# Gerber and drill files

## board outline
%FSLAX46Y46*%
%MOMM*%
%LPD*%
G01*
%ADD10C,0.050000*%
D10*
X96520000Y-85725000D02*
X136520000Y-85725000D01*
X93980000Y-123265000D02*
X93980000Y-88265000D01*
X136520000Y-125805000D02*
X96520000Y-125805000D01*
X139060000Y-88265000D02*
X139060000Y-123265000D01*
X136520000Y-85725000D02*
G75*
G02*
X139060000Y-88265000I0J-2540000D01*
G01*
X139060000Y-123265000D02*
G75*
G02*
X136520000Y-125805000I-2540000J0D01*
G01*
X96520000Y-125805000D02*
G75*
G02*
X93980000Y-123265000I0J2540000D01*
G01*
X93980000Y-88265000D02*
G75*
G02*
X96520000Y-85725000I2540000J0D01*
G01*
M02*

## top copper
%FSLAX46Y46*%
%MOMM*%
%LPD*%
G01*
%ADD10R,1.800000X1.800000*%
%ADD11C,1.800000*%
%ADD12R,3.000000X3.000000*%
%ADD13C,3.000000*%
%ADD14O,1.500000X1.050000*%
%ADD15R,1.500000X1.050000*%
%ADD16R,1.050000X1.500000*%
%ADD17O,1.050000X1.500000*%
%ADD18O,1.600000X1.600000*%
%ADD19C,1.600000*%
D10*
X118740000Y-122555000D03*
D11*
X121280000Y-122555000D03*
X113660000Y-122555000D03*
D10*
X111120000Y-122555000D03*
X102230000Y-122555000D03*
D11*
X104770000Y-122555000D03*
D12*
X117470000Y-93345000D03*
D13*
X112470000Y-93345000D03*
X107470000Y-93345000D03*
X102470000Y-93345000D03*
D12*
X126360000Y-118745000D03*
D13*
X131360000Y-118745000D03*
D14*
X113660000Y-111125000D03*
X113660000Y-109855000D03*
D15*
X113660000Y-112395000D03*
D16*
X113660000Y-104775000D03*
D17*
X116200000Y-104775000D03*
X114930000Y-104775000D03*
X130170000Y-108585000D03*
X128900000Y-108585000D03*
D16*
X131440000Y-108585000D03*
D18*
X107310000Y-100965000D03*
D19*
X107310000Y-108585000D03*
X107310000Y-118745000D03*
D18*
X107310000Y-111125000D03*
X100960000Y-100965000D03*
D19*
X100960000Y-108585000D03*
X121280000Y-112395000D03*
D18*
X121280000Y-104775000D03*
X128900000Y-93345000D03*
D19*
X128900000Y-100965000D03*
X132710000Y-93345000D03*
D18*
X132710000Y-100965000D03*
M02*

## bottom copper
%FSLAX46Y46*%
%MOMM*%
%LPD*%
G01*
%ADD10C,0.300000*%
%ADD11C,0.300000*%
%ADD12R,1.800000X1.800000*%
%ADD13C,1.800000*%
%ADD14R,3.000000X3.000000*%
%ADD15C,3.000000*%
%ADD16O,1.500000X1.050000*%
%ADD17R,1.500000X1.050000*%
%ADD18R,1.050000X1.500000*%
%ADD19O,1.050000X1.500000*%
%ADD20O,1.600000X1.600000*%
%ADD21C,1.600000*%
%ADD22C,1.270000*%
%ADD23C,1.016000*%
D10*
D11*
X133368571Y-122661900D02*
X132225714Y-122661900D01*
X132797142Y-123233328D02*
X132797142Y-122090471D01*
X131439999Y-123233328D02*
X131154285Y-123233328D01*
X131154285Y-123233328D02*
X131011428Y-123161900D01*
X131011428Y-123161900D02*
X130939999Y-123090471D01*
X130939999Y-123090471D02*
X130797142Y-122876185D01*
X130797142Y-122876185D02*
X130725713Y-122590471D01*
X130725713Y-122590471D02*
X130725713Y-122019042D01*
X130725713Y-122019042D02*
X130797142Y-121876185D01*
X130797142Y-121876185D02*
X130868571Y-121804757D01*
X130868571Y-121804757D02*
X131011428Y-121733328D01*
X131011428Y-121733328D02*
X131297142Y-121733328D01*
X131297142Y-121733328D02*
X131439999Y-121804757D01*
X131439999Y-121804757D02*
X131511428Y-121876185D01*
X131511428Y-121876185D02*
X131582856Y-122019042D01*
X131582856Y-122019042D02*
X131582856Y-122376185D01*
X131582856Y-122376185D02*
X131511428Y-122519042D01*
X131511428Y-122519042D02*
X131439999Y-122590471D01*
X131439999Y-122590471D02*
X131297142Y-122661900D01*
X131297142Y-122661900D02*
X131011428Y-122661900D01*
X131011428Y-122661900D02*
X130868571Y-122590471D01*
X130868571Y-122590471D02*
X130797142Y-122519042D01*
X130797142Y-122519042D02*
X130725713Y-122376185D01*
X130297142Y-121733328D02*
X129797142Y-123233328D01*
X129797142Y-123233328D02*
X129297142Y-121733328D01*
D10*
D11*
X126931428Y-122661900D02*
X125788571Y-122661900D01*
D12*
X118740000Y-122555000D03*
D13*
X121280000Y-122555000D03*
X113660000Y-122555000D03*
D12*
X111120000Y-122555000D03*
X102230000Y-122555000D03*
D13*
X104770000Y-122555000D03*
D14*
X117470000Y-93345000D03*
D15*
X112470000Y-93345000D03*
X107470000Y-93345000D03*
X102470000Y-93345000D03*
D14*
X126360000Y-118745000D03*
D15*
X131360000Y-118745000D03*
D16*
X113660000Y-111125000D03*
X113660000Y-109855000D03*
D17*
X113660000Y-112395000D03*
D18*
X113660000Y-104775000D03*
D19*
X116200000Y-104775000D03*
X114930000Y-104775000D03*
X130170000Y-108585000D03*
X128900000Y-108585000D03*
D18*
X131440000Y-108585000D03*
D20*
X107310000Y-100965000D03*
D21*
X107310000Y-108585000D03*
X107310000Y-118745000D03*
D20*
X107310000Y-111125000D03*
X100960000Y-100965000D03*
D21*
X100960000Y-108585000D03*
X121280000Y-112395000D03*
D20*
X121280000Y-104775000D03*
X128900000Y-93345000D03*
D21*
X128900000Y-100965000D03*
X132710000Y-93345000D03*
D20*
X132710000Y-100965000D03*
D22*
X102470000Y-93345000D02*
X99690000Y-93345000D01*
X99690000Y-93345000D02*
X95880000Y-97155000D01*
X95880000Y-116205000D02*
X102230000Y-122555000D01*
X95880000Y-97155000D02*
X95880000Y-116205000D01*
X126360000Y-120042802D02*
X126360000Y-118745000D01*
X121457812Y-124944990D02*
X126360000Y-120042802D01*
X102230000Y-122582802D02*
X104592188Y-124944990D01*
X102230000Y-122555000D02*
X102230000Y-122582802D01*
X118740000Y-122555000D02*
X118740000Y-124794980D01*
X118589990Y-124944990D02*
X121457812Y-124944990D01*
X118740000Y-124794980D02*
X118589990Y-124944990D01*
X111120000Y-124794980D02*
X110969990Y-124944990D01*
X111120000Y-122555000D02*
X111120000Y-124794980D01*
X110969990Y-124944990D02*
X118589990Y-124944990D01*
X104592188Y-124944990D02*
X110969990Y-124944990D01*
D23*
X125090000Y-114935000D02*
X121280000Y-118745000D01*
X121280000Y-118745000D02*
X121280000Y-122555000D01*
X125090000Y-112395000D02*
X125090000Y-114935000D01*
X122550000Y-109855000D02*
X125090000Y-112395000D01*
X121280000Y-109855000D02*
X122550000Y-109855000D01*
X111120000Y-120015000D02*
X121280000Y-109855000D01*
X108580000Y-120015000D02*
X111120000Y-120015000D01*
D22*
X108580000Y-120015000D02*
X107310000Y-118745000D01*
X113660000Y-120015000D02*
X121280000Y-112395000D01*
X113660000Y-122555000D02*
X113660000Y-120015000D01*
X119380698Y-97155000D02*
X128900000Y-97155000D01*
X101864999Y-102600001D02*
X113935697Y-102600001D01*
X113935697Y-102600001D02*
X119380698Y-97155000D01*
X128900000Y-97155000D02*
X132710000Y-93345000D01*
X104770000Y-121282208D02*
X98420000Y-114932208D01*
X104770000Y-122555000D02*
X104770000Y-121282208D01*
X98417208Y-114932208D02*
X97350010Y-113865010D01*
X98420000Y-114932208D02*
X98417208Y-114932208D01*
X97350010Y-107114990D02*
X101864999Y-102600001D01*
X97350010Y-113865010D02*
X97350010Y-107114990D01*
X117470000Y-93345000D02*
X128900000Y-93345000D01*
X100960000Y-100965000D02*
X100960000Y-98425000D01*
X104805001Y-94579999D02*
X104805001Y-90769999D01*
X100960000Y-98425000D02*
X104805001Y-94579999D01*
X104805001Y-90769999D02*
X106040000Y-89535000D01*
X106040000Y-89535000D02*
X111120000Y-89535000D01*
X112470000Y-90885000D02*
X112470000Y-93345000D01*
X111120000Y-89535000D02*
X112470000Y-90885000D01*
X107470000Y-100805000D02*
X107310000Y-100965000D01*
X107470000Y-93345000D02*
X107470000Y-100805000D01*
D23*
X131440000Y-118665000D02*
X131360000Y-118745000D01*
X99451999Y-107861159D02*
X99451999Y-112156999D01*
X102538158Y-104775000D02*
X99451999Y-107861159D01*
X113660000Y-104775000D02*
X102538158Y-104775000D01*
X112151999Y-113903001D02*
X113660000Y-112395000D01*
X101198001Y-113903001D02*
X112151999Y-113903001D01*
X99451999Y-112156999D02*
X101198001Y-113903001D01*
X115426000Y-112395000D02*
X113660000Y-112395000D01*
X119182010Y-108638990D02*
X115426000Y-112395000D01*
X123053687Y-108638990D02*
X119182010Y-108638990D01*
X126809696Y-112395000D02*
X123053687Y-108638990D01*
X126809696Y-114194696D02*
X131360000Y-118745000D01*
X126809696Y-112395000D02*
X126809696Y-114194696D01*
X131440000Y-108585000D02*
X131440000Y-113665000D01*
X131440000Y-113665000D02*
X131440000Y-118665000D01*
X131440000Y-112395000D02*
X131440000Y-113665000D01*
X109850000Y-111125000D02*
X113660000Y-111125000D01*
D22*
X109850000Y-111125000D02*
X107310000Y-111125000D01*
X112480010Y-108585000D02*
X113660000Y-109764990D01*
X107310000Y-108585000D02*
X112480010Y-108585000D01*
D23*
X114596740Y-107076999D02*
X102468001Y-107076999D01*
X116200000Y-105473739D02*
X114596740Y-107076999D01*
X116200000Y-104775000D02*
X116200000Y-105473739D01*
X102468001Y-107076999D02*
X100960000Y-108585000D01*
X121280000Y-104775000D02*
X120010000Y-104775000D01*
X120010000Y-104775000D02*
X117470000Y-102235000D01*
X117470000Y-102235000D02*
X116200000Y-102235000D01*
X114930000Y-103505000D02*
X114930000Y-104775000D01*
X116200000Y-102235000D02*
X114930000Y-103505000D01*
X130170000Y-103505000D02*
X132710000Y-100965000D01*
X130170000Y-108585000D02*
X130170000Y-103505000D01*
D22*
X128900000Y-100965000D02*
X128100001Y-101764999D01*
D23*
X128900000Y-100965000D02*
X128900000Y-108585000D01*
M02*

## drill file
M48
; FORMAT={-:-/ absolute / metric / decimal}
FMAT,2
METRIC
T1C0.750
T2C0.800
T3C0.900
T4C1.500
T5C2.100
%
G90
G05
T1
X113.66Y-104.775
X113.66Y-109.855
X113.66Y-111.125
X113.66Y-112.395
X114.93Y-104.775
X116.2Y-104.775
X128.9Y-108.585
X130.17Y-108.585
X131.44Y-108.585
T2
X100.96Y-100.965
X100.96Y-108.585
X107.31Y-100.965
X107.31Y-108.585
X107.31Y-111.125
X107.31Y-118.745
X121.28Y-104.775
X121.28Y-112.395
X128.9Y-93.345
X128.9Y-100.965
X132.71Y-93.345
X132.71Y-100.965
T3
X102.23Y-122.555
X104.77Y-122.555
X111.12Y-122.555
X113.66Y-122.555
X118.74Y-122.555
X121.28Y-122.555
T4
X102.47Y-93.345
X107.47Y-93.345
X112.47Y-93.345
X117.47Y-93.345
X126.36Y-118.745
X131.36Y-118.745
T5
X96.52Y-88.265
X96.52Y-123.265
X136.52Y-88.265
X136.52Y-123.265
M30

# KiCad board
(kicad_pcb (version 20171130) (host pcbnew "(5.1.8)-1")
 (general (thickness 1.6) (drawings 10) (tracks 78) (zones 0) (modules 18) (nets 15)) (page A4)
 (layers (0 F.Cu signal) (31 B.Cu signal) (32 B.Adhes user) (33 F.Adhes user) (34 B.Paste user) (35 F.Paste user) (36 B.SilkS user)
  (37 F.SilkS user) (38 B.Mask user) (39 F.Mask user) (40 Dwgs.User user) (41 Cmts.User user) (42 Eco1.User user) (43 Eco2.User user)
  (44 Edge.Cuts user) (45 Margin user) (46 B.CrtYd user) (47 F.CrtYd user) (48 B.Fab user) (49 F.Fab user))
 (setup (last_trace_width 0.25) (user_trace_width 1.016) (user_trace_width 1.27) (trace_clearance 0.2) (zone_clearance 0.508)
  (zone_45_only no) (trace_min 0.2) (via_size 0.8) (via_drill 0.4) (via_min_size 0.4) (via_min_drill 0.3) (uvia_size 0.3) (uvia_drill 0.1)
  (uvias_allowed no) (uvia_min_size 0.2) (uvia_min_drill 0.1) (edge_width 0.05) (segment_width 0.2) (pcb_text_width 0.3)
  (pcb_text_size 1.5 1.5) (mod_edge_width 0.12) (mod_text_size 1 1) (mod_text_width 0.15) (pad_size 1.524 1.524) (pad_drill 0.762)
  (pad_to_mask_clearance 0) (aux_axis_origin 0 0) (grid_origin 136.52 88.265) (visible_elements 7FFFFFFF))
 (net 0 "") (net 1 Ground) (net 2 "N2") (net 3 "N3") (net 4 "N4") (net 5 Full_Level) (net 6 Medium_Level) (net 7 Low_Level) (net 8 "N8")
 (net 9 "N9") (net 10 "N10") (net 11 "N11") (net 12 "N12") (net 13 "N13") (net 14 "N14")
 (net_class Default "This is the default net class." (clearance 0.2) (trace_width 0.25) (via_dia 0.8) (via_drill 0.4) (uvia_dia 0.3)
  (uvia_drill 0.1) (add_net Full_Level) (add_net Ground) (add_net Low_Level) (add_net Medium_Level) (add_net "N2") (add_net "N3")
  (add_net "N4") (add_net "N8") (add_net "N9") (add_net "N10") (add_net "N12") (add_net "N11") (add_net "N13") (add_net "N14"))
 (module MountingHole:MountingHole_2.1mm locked (layer F.Cu) (at 136.52 123.265)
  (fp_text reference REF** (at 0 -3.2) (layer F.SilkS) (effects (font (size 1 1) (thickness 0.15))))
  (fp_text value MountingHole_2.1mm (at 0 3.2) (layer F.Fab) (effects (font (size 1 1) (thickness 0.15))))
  (pad "" np_thru_hole circle (at 0 0) (size 2.1 2.1) (drill 2.1) (layers *.Cu *.Mask)))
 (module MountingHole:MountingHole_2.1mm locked (layer F.Cu) (at 96.52 123.265)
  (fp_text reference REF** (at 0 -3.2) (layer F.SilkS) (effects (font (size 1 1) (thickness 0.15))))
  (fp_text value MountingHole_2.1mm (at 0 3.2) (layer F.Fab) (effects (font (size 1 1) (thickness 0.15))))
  (pad "" np_thru_hole circle (at 0 0) (size 2.1 2.1) (drill 2.1) (layers *.Cu *.Mask)))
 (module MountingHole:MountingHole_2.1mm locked (layer F.Cu) (at 136.52 88.265)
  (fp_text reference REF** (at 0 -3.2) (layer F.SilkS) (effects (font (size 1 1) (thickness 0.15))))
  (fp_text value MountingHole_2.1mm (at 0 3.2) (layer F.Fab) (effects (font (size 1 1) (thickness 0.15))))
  (pad "" np_thru_hole circle (at 0 0) (size 2.1 2.1) (drill 2.1) (layers *.Cu *.Mask)))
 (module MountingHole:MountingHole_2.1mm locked (layer F.Cu) (at 96.52 88.265)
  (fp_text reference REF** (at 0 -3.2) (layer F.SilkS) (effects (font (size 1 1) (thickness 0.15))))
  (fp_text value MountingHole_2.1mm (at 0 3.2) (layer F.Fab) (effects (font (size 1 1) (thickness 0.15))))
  (pad "" np_thru_hole circle (at 0 0) (size 2.1 2.1) (drill 2.1) (layers *.Cu *.Mask)))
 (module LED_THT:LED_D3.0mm (layer F.Cu) (at 118.74 122.555)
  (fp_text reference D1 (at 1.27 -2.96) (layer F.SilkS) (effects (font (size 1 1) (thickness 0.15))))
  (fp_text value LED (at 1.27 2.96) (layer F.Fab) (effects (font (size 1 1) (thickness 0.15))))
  (pad 1 thru_hole rect (at 0 0) (size 1.8 1.8) (drill 0.9) (layers *.Cu *.Mask) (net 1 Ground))
  (pad 2 thru_hole circle (at 2.54 0) (size 1.8 1.8) (drill 0.9) (layers *.Cu *.Mask) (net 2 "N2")))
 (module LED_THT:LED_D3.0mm (layer F.Cu) (at 111.12 122.555)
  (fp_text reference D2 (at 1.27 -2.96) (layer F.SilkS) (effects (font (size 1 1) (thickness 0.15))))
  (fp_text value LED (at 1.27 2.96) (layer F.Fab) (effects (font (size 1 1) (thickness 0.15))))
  (pad 2 thru_hole circle (at 2.54 0) (size 1.8 1.8) (drill 0.9) (layers *.Cu *.Mask) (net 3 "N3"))
  (pad 1 thru_hole rect (at 0 0) (size 1.8 1.8) (drill 0.9) (layers *.Cu *.Mask) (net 1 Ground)))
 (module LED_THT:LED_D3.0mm (layer F.Cu) (at 102.23 122.555)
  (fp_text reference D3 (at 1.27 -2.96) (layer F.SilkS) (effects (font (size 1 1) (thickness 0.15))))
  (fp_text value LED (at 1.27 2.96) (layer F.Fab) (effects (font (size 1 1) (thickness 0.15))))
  (pad 1 thru_hole rect (at 0 0) (size 1.8 1.8) (drill 0.9) (layers *.Cu *.Mask) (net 1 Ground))
  (pad 2 thru_hole circle (at 2.54 0) (size 1.8 1.8) (drill 0.9) (layers *.Cu *.Mask) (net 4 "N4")))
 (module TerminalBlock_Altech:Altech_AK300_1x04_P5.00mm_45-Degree (layer F.Cu) (at 117.47 93.345 180)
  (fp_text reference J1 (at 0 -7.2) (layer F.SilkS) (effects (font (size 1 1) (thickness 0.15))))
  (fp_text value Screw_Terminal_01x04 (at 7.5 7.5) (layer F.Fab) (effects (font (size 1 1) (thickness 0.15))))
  (pad 1 thru_hole rect (at 0 0 180) (size 3 3) (drill 1.5) (layers *.Cu *.Mask) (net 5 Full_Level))
  (pad 2 thru_hole circle (at 5 0 180) (size 3 3) (drill 1.5) (layers *.Cu *.Mask) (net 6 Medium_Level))
  (pad 3 thru_hole circle (at 10 0 180) (size 3 3) (drill 1.5) (layers *.Cu *.Mask) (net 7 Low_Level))
  (pad 4 thru_hole circle (at 15 0 180) (size 3 3) (drill 1.5) (layers *.Cu *.Mask) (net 1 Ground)))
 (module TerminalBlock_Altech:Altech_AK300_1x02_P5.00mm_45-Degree (layer F.Cu) (at 126.36 118.745)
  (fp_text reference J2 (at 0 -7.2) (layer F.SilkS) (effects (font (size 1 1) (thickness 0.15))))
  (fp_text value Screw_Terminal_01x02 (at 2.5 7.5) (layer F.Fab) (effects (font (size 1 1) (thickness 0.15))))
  (pad 1 thru_hole rect (at 0 0) (size 3 3) (drill 1.5) (layers *.Cu *.Mask) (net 1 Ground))
  (pad 2 thru_hole circle (at 5 0) (size 3 3) (drill 1.5) (layers *.Cu *.Mask) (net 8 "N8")))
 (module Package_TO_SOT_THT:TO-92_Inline (layer F.Cu) (at 113.66 112.395 90)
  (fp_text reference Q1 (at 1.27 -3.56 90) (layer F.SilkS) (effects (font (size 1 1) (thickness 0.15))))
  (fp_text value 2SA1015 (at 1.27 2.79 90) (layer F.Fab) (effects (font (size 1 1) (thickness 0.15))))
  (pad 2 thru_hole oval (at 1.27 0 90) (size 1.05 1.5) (drill 0.75) (layers *.Cu *.Mask) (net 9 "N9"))
  (pad 3 thru_hole oval (at 2.54 0 90) (size 1.05 1.5) (drill 0.75) (layers *.Cu *.Mask) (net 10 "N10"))
  (pad 1 thru_hole rect (at 0 0 90) (size 1.05 1.5) (drill 0.75) (layers *.Cu *.Mask) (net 8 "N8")))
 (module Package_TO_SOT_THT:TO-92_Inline (layer F.Cu) (at 113.66 104.775)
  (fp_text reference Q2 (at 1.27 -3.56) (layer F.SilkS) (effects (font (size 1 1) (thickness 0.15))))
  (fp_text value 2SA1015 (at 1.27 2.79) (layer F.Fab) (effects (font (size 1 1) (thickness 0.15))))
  (pad 1 thru_hole rect (at 0 0) (size 1.05 1.5) (drill 0.75) (layers *.Cu *.Mask) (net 8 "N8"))
  (pad 3 thru_hole oval (at 2.54 0) (size 1.05 1.5) (drill 0.75) (layers *.Cu *.Mask) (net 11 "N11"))
  (pad 2 thru_hole oval (at 1.27 0) (size 1.05 1.5) (drill 0.75) (layers *.Cu *.Mask) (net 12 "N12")))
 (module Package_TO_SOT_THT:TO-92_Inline (layer F.Cu) (at 131.44 108.585 180)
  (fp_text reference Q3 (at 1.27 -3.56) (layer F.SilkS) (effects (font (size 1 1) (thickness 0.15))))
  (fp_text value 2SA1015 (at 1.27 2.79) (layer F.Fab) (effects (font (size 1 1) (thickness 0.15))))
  (pad 2 thru_hole oval (at 1.27 0 180) (size 1.05 1.5) (drill 0.75) (layers *.Cu *.Mask) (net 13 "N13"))
  (pad 3 thru_hole oval (at 2.54 0 180) (size 1.05 1.5) (drill 0.75) (layers *.Cu *.Mask) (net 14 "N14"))
  (pad 1 thru_hole rect (at 0 0 180) (size 1.05 1.5) (drill 0.75) (layers *.Cu *.Mask) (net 8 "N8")))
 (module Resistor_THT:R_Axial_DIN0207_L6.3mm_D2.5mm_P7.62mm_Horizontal (layer F.Cu) (at 107.31 108.585 90)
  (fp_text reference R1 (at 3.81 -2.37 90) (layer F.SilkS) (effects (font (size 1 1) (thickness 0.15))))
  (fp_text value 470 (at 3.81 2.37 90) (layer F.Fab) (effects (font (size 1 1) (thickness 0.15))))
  (pad 2 thru_hole oval (at 7.62 0 90) (size 1.6 1.6) (drill 0.8) (layers *.Cu *.Mask) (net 7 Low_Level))
  (pad 1 thru_hole circle (at 0 0 90) (size 1.6 1.6) (drill 0.8) (layers *.Cu *.Mask) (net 10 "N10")))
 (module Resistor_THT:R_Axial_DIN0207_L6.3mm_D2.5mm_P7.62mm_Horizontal (layer F.Cu) (at 107.31 118.745 90)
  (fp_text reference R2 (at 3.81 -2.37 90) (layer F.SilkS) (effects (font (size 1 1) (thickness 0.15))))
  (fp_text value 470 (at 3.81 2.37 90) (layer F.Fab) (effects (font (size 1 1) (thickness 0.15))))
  (pad 1 thru_hole circle (at 0 0 90) (size 1.6 1.6) (drill 0.8) (layers *.Cu *.Mask) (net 2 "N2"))
  (pad 2 thru_hole oval (at 7.62 0 90) (size 1.6 1.6) (drill 0.8) (layers *.Cu *.Mask) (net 9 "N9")))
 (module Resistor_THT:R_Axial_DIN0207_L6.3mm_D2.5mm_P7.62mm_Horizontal (layer F.Cu) (at 100.96 108.585 90)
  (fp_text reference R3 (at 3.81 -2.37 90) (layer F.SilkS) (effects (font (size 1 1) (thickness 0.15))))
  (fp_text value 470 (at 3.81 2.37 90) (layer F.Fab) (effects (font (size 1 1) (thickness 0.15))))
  (pad 2 thru_hole oval (at 7.62 0 90) (size 1.6 1.6) (drill 0.8) (layers *.Cu *.Mask) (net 6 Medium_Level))
  (pad 1 thru_hole circle (at 0 0 90) (size 1.6 1.6) (drill 0.8) (layers *.Cu *.Mask) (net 11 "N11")))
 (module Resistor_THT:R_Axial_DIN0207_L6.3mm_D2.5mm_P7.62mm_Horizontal (layer F.Cu) (at 121.28 112.395 90)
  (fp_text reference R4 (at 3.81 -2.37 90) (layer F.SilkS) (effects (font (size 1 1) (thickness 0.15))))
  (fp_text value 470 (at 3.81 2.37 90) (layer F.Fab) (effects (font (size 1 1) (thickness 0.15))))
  (pad 1 thru_hole circle (at 0 0 90) (size 1.6 1.6) (drill 0.8) (layers *.Cu *.Mask) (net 3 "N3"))
  (pad 2 thru_hole oval (at 7.62 0 90) (size 1.6 1.6) (drill 0.8) (layers *.Cu *.Mask) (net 12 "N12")))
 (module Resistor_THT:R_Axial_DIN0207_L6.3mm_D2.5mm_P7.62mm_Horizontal (layer F.Cu) (at 128.9 100.965 90)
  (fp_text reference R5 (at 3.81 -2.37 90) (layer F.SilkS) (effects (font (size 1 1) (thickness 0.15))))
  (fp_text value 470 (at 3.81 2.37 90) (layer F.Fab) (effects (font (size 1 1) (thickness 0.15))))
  (pad 2 thru_hole oval (at 7.62 0 90) (size 1.6 1.6) (drill 0.8) (layers *.Cu *.Mask) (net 5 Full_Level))
  (pad 1 thru_hole circle (at 0 0 90) (size 1.6 1.6) (drill 0.8) (layers *.Cu *.Mask) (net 14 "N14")))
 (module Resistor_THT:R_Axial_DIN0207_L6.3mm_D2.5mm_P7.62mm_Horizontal (layer F.Cu) (at 132.71 93.345 270)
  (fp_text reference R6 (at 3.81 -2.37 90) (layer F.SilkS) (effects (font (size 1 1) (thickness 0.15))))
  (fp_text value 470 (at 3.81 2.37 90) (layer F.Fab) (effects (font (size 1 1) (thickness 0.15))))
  (pad 1 thru_hole circle (at 0 0 270) (size 1.6 1.6) (drill 0.8) (layers *.Cu *.Mask) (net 4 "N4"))
  (pad 2 thru_hole oval (at 7.62 0 270) (size 1.6 1.6) (drill 0.8) (layers *.Cu *.Mask) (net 13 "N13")))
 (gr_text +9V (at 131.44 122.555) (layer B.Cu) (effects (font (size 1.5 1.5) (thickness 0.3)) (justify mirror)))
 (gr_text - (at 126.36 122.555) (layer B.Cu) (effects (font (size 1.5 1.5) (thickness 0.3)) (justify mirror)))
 (gr_line (start 96.52 85.725) (end 136.52 85.725) (layer Edge.Cuts) (width 0.05))
 (gr_line (start 93.98 123.265) (end 93.98 88.265) (layer Edge.Cuts) (width 0.05))
 (gr_line (start 136.52 125.805) (end 96.52 125.805) (layer Edge.Cuts) (width 0.05))
 (gr_line (start 139.06 88.265) (end 139.06 123.265) (layer Edge.Cuts) (width 0.05))
 (gr_arc (start 136.52 88.265) (end 139.06 88.265) (angle -90) (layer Edge.Cuts) (width 0.05))
 (gr_arc (start 136.52 123.265) (end 136.52 125.805) (angle -90) (layer Edge.Cuts) (width 0.05))
 (gr_arc (start 96.52 123.265) (end 93.98 123.265) (angle -90) (layer Edge.Cuts) (width 0.05))
 (gr_arc (start 96.52 88.265) (end 96.52 85.725) (angle -90) (layer Edge.Cuts) (width 0.05))
 (segment (start 102.47 93.345) (end 99.69 93.345) (width 1.27) (layer B.Cu) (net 1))
 (segment (start 99.69 93.345) (end 95.88 97.155) (width 1.27) (layer B.Cu) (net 1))
 (segment (start 95.88 116.205) (end 102.23 122.555) (width 1.27) (layer B.Cu) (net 1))
 (segment (start 95.88 97.155) (end 95.88 116.205) (width 1.27) (layer B.Cu) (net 1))
 (segment (start 126.36 120.042802) (end 126.36 118.745) (width 1.27) (layer B.Cu) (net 1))
 (segment (start 121.457812 124.94499) (end 126.36 120.042802) (width 1.27) (layer B.Cu) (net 1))
 (segment (start 102.23 122.582802) (end 104.592188 124.94499) (width 1.27) (layer B.Cu) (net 1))
 (segment (start 102.23 122.555) (end 102.23 122.582802) (width 1.27) (layer B.Cu) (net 1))
 (segment (start 118.74 122.555) (end 118.74 124.79498) (width 1.27) (layer B.Cu) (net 1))
 (segment (start 118.58999 124.94499) (end 121.457812 124.94499) (width 1.27) (layer B.Cu) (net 1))
 (segment (start 118.74 124.79498) (end 118.58999 124.94499) (width 1.27) (layer B.Cu) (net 1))
 (segment (start 111.12 124.79498) (end 110.96999 124.94499) (width 1.27) (layer B.Cu) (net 1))
 (segment (start 111.12 122.555) (end 111.12 124.79498) (width 1.27) (layer B.Cu) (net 1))
 (segment (start 110.96999 124.94499) (end 118.58999 124.94499) (width 1.27) (layer B.Cu) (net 1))
 (segment (start 104.592188 124.94499) (end 110.96999 124.94499) (width 1.27) (layer B.Cu) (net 1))
 (segment (start 125.09 114.935) (end 121.28 118.745) (width 1.016) (layer B.Cu) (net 2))
 (segment (start 121.28 118.745) (end 121.28 122.555) (width 1.016) (layer B.Cu) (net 2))
 (segment (start 125.09 112.395) (end 125.09 114.935) (width 1.016) (layer B.Cu) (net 2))
 (segment (start 122.55 109.855) (end 125.09 112.395) (width 1.016) (layer B.Cu) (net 2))
 (segment (start 121.28 109.855) (end 122.55 109.855) (width 1.016) (layer B.Cu) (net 2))
 (segment (start 111.12 120.015) (end 121.28 109.855) (width 1.016) (layer B.Cu) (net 2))
 (segment (start 108.58 120.015) (end 111.12 120.015) (width 1.016) (layer B.Cu) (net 2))
 (segment (start 108.58 120.015) (end 107.31 118.745) (width 1.27) (layer B.Cu) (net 2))
 (segment (start 113.66 120.015) (end 121.28 112.395) (width 1.27) (layer B.Cu) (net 3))
 (segment (start 113.66 122.555) (end 113.66 120.015) (width 1.27) (layer B.Cu) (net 3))
 (segment (start 119.380698 97.155) (end 128.9 97.155) (width 1.27) (layer B.Cu) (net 4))
 (segment (start 101.864999 102.600001) (end 113.935697 102.600001) (width 1.27) (layer B.Cu) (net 4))
 (segment (start 113.935697 102.600001) (end 119.380698 97.155) (width 1.27) (layer B.Cu) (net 4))
 (segment (start 128.9 97.155) (end 132.71 93.345) (width 1.27) (layer B.Cu) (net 4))
 (segment (start 104.77 121.282208) (end 98.42 114.932208) (width 1.27) (layer B.Cu) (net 4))
 (segment (start 104.77 122.555) (end 104.77 121.282208) (width 1.27) (layer B.Cu) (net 4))
 (segment (start 98.417208 114.932208) (end 97.35001 113.86501) (width 1.27) (layer B.Cu) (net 4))
 (segment (start 98.42 114.932208) (end 98.417208 114.932208) (width 1.27) (layer B.Cu) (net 4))
 (segment (start 97.35001 107.11499) (end 101.864999 102.600001) (width 1.27) (layer B.Cu) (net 4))
 (segment (start 97.35001 113.86501) (end 97.35001 107.11499) (width 1.27) (layer B.Cu) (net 4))
 (segment (start 117.47 93.345) (end 128.9 93.345) (width 1.27) (layer B.Cu) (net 5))
 (segment (start 100.96 100.965) (end 100.96 98.425) (width 1.27) (layer B.Cu) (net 6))
 (segment (start 104.805001 94.579999) (end 104.805001 90.769999) (width 1.27) (layer B.Cu) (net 6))
 (segment (start 100.96 98.425) (end 104.805001 94.579999) (width 1.27) (layer B.Cu) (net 6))
 (segment (start 104.805001 90.769999) (end 106.04 89.535) (width 1.27) (layer B.Cu) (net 6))
 (segment (start 106.04 89.535) (end 111.12 89.535) (width 1.27) (layer B.Cu) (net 6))
 (segment (start 112.47 90.885) (end 112.47 93.345) (width 1.27) (layer B.Cu) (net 6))
 (segment (start 111.12 89.535) (end 112.47 90.885) (width 1.27) (layer B.Cu) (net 6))
 (segment (start 107.47 100.805) (end 107.31 100.965) (width 1.27) (layer B.Cu) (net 7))
 (segment (start 107.47 93.345) (end 107.47 100.805) (width 1.27) (layer B.Cu) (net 7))
 (segment (start 131.44 118.665) (end 131.36 118.745) (width 1.016) (layer B.Cu) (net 8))
 (segment (start 99.451999 107.861159) (end 99.451999 112.156999) (width 1.016) (layer B.Cu) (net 8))
 (segment (start 102.538158 104.775) (end 99.451999 107.861159) (width 1.016) (layer B.Cu) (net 8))
 (segment (start 113.66 104.775) (end 102.538158 104.775) (width 1.016) (layer B.Cu) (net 8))
 (segment (start 112.151999 113.903001) (end 113.66 112.395) (width 1.016) (layer B.Cu) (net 8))
 (segment (start 101.198001 113.903001) (end 112.151999 113.903001) (width 1.016) (layer B.Cu) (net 8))
 (segment (start 99.451999 112.156999) (end 101.198001 113.903001) (width 1.016) (layer B.Cu) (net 8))
 (segment (start 115.426 112.395) (end 113.66 112.395) (width 1.016) (layer B.Cu) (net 8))
 (segment (start 119.18201 108.63899) (end 115.426 112.395) (width 1.016) (layer B.Cu) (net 8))
 (segment (start 123.053687 108.63899) (end 119.18201 108.63899) (width 1.016) (layer B.Cu) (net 8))
 (segment (start 126.809696 112.395) (end 123.053687 108.63899) (width 1.016) (layer B.Cu) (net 8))
 (segment (start 126.809696 114.194696) (end 131.36 118.745) (width 1.016) (layer B.Cu) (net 8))
 (segment (start 126.809696 112.395) (end 126.809696 114.194696) (width 1.016) (layer B.Cu) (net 8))
 (segment (start 131.44 108.585) (end 131.44 113.665) (width 1.016) (layer B.Cu) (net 8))
 (segment (start 131.44 113.665) (end 131.44 118.665) (width 1.016) (layer B.Cu) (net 8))
 (segment (start 131.44 112.395) (end 131.44 113.665) (width 1.016) (layer B.Cu) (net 8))
 (segment (start 109.85 111.125) (end 113.66 111.125) (width 1.016) (layer B.Cu) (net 9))
 (segment (start 109.85 111.125) (end 107.31 111.125) (width 1.27) (layer B.Cu) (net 9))
 (segment (start 112.48001 108.585) (end 113.66 109.76499) (width 1.27) (layer B.Cu) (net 10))
 (segment (start 107.31 108.585) (end 112.48001 108.585) (width 1.27) (layer B.Cu) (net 10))
 (segment (start 114.59674 107.076999) (end 102.468001 107.076999) (width 1.016) (layer B.Cu) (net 11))
 (segment (start 116.2 105.473739) (end 114.59674 107.076999) (width 1.016) (layer B.Cu) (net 11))
 (segment (start 116.2 104.775) (end 116.2 105.473739) (width 1.016) (layer B.Cu) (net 11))
 (segment (start 102.468001 107.076999) (end 100.96 108.585) (width 1.016) (layer B.Cu) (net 11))
 (segment (start 121.28 104.775) (end 120.01 104.775) (width 1.016) (layer B.Cu) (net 12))
 (segment (start 120.01 104.775) (end 117.47 102.235) (width 1.016) (layer B.Cu) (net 12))
 (segment (start 117.47 102.235) (end 116.2 102.235) (width 1.016) (layer B.Cu) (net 12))
 (segment (start 114.93 103.505) (end 114.93 104.775) (width 1.016) (layer B.Cu) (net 12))
 (segment (start 116.2 102.235) (end 114.93 103.505) (width 1.016) (layer B.Cu) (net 12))
 (segment (start 130.17 103.505) (end 132.71 100.965) (width 1.016) (layer B.Cu) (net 13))
 (segment (start 130.17 108.585) (end 130.17 103.505) (width 1.016) (layer B.Cu) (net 13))
 (segment (start 128.9 100.965) (end 128.100001 101.764999) (width 1.27) (layer B.Cu) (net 14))
 (segment (start 128.9 100.965) (end 128.9 108.585) (width 1.016) (layer B.Cu) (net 14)))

